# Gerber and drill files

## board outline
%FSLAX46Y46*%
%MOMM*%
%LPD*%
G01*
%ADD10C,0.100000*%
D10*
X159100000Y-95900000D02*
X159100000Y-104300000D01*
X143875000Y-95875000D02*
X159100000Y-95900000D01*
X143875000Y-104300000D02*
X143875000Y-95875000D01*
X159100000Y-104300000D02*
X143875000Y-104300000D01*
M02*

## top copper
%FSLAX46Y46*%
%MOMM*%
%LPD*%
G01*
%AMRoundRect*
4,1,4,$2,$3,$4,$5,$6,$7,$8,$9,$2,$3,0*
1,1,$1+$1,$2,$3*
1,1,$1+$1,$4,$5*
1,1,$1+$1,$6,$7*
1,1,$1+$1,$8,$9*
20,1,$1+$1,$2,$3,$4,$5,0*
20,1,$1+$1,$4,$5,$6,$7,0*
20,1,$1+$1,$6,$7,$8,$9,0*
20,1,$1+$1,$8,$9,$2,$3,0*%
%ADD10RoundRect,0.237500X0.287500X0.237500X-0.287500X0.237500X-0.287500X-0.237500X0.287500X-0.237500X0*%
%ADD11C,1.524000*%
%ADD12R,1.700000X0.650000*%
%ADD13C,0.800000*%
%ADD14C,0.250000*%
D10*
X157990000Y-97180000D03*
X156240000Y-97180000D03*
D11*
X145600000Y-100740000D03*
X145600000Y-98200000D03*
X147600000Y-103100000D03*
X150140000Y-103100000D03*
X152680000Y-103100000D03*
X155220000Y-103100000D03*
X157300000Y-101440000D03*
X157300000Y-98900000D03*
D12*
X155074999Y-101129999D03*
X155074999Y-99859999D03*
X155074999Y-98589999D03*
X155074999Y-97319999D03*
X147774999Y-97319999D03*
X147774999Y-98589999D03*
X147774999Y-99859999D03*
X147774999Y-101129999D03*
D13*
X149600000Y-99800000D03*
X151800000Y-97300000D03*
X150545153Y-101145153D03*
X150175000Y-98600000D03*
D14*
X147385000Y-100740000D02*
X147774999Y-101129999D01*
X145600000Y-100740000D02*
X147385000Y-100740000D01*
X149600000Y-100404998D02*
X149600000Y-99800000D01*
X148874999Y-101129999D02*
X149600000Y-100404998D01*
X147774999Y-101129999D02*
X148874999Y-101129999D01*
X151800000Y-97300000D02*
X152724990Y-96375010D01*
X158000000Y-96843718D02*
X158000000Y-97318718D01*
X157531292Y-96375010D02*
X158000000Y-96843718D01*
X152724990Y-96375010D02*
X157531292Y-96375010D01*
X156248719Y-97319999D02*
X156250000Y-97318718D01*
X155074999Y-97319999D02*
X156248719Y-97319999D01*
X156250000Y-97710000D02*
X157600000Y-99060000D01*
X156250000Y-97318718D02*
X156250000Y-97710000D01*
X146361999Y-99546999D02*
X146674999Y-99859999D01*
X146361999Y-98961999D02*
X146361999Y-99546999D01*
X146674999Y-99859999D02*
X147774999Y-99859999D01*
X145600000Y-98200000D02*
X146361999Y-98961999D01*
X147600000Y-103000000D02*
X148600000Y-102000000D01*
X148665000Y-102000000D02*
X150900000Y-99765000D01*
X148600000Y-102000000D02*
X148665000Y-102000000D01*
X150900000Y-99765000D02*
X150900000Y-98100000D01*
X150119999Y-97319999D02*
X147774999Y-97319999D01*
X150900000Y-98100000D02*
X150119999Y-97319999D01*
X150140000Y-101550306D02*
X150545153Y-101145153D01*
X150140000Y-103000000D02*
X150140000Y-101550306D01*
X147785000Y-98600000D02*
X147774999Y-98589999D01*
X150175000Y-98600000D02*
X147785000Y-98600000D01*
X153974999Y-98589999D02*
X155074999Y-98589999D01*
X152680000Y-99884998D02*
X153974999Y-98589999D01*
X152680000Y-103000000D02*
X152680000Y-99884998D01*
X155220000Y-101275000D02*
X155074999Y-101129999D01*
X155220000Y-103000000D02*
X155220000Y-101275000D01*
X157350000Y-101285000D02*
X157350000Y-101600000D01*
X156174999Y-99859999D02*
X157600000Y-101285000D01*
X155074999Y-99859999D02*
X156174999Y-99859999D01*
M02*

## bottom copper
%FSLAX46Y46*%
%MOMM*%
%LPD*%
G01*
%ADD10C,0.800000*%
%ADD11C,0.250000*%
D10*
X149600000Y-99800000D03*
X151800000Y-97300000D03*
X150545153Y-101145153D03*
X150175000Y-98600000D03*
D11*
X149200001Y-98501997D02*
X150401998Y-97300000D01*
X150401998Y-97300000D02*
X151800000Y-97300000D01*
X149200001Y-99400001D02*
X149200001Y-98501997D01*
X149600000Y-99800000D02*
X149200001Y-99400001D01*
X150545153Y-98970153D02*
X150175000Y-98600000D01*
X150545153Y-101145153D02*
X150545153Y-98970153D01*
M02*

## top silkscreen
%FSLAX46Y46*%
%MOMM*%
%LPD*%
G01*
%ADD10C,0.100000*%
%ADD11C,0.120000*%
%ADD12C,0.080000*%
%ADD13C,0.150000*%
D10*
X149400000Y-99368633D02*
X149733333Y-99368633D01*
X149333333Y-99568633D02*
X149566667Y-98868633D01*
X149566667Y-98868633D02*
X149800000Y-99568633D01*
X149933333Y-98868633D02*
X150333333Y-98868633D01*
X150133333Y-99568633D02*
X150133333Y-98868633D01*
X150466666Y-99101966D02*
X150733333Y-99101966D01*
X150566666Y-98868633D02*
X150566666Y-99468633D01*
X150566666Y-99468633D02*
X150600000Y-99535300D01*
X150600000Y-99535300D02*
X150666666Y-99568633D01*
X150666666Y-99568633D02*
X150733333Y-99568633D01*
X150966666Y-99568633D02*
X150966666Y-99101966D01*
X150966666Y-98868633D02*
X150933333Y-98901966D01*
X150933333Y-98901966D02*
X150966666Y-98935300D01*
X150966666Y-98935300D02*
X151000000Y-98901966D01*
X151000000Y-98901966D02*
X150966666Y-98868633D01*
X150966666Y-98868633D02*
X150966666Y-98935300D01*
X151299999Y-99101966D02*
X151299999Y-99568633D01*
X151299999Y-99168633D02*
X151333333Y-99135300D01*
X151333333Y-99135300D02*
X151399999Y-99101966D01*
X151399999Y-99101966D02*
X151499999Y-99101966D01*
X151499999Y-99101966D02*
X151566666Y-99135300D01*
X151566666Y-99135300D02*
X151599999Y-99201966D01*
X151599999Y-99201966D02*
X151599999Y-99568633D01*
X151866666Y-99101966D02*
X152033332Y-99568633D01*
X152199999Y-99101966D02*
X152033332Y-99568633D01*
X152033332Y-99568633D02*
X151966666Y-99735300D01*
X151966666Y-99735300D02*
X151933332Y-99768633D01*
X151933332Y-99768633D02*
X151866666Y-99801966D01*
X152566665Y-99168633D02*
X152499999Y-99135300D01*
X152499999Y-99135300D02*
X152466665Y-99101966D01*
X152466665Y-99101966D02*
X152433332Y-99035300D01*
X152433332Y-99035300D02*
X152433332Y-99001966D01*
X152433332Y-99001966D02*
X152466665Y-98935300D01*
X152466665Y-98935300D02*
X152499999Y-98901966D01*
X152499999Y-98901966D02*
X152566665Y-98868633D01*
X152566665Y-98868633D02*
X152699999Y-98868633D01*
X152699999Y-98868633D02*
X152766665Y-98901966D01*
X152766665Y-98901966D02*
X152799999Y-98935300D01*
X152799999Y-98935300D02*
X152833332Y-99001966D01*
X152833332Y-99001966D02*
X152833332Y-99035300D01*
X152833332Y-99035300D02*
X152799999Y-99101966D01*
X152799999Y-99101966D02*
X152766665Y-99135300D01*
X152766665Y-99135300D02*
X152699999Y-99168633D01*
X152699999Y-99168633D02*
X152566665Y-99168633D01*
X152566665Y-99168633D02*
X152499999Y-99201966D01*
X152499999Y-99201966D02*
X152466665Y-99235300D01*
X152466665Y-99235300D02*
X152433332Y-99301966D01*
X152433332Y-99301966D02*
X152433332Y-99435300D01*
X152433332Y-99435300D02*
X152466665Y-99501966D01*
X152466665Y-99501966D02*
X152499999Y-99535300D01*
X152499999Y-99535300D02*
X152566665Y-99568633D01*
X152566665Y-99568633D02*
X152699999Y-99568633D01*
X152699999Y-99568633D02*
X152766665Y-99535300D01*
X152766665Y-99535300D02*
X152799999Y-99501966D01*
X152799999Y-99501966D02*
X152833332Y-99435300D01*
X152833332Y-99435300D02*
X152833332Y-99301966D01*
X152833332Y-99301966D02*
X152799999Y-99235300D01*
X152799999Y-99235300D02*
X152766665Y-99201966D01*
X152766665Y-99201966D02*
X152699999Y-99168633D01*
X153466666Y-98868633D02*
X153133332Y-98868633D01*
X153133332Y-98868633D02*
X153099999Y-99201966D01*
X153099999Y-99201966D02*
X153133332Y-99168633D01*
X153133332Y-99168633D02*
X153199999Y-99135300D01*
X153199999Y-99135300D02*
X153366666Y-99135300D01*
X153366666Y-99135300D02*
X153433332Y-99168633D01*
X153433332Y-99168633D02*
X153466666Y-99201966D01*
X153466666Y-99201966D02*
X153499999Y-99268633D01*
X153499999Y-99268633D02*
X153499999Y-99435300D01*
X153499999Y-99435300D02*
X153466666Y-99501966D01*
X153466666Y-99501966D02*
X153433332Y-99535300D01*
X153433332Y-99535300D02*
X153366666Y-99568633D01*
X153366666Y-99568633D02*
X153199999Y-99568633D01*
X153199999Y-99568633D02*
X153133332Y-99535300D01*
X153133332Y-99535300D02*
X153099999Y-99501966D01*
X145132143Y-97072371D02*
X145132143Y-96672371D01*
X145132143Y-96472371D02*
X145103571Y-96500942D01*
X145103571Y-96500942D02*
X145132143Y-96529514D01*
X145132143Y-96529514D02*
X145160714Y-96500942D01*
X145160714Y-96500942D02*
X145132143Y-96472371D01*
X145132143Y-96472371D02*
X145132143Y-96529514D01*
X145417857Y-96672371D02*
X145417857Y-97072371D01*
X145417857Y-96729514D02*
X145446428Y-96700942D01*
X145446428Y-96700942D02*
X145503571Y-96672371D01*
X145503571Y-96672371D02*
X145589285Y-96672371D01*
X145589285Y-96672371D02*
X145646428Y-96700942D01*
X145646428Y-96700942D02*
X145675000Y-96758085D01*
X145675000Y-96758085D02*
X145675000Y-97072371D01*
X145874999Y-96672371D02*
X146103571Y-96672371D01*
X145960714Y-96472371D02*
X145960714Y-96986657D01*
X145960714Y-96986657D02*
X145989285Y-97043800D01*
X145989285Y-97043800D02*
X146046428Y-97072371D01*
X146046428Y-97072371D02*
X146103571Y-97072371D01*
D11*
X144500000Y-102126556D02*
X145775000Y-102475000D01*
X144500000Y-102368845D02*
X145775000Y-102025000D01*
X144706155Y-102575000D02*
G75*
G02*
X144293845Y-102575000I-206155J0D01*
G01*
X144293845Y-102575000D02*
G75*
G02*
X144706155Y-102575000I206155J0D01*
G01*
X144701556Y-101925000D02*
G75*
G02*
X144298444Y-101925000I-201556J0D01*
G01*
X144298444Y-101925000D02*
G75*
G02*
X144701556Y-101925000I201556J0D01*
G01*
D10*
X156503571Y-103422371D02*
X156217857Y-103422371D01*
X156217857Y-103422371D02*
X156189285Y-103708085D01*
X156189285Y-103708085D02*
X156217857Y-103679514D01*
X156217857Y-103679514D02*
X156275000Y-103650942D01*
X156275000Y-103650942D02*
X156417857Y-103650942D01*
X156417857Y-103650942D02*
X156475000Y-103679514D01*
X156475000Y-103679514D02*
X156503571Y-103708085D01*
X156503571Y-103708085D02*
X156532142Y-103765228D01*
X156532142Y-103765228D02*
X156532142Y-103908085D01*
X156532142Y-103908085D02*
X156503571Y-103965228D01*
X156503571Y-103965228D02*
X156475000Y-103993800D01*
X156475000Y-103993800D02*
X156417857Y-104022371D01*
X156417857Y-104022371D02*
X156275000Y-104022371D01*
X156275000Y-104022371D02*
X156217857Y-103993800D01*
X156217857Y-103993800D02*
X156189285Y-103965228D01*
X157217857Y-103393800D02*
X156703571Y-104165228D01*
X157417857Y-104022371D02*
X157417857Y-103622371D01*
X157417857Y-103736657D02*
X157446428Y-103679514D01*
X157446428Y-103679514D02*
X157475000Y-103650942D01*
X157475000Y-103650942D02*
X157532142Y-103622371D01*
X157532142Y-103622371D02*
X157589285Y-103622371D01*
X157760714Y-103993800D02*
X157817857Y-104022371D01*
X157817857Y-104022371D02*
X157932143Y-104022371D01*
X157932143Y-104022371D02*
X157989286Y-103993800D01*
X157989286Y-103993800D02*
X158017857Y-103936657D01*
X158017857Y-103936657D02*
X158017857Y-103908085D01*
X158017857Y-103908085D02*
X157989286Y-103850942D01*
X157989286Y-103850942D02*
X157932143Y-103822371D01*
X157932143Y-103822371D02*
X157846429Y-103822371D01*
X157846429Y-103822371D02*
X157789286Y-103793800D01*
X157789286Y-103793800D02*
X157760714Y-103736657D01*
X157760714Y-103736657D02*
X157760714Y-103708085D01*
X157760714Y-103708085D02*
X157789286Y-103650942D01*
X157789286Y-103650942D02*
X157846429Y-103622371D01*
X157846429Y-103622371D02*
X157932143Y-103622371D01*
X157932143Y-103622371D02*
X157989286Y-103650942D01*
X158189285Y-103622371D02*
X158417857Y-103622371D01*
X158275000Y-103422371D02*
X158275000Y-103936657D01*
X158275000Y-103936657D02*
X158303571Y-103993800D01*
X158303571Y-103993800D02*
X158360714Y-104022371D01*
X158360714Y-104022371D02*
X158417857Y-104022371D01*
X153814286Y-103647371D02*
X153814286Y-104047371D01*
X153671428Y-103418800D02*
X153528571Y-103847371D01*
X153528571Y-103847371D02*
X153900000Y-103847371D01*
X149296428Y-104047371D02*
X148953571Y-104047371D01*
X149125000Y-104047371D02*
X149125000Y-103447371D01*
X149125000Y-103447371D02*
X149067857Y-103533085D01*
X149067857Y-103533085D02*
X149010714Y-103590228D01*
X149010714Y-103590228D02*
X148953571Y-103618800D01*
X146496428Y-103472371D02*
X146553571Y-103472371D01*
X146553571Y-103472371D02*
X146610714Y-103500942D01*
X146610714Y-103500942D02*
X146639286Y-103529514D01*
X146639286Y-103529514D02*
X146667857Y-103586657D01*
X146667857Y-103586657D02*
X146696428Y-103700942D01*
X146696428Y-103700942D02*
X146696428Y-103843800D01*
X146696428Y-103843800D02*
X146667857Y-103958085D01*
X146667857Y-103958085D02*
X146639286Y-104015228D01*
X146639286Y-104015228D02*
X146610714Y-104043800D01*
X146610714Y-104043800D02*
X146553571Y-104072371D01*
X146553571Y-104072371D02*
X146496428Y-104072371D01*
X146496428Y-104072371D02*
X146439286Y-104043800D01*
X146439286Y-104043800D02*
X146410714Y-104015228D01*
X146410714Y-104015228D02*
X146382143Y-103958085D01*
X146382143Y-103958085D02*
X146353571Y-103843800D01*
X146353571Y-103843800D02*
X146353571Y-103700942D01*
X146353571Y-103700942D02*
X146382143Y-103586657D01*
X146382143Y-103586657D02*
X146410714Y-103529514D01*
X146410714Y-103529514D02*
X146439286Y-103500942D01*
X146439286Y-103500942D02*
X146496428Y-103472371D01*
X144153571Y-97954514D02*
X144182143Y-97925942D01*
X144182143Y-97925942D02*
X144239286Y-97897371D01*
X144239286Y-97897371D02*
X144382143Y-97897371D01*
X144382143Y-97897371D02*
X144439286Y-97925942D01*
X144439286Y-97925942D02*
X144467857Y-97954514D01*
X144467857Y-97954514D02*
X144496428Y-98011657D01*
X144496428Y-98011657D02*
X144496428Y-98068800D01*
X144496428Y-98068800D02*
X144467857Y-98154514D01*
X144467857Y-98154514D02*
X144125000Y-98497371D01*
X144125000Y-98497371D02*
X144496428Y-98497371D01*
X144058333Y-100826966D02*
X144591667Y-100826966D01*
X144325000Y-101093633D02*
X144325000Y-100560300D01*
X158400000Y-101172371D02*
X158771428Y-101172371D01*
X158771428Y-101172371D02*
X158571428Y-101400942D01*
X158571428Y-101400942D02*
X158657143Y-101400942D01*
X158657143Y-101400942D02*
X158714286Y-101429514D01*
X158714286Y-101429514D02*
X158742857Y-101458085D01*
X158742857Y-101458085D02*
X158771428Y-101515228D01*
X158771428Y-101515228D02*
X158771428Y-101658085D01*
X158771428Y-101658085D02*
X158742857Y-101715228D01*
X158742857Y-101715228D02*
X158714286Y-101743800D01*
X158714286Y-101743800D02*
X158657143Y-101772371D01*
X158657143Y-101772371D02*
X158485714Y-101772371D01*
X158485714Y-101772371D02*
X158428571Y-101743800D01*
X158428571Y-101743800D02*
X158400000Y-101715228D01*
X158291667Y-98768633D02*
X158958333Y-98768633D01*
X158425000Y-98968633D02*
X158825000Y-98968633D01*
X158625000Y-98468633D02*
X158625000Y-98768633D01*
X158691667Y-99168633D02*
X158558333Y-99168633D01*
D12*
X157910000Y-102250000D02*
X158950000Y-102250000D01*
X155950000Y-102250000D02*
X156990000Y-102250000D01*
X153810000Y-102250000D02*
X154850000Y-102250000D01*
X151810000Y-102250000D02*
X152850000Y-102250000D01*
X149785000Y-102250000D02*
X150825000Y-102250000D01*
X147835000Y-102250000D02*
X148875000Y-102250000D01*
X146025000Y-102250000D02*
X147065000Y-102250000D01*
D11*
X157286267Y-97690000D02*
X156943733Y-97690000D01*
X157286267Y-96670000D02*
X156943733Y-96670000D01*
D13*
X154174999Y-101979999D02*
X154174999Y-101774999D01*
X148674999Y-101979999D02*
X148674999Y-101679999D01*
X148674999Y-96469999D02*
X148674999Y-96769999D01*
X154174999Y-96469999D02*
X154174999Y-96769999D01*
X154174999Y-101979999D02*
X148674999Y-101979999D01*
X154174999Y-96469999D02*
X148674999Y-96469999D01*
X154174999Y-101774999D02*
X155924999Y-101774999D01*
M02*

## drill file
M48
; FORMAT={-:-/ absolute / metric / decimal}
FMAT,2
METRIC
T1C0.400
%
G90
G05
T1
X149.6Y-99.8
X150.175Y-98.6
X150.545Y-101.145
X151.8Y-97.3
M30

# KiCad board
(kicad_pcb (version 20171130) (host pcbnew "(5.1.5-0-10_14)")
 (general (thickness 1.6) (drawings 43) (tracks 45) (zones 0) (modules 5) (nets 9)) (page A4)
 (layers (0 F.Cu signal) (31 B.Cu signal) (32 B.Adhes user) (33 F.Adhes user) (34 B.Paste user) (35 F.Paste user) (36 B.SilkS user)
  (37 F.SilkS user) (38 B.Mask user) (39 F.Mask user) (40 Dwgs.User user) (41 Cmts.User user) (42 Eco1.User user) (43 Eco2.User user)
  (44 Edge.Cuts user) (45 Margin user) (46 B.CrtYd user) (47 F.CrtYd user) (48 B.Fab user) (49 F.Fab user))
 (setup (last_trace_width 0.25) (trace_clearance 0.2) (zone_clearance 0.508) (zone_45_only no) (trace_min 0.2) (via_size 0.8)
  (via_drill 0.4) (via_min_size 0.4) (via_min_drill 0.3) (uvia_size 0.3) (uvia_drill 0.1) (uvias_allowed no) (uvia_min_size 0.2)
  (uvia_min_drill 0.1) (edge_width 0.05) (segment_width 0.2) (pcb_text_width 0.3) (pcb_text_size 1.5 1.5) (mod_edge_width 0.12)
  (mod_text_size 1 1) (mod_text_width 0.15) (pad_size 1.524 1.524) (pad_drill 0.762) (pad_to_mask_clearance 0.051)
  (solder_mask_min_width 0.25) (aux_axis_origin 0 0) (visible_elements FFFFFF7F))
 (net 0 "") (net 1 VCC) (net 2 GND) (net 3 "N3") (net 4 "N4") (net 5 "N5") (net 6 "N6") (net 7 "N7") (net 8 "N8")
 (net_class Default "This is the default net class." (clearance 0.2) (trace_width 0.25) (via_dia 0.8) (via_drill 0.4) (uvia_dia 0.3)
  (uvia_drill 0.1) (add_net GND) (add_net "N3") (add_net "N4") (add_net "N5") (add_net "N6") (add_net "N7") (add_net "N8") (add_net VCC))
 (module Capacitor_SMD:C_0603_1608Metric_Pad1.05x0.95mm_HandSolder (layer F.Cu) (at 157.115 97.18 180)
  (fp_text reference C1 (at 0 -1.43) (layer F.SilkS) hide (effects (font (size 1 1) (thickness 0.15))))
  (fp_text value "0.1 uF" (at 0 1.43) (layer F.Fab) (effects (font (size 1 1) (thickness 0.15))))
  (fp_line (start -0.171267 -0.51) (end 0.171267 -0.51) (layer F.SilkS) (width 0.12))
  (fp_line (start -0.171267 0.51) (end 0.171267 0.51) (layer F.SilkS) (width 0.12))
  (pad 1 smd roundrect (at -0.875 0 180) (size 1.05 0.95) (layers F.Cu F.Paste F.Mask) (roundrect_rratio 0.25) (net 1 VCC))
  (pad 2 smd roundrect (at 0.875 0 180) (size 1.05 0.95) (layers F.Cu F.Paste F.Mask) (roundrect_rratio 0.25) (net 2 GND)))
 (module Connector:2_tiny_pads (layer F.Cu) (at 143.06 99.47 90)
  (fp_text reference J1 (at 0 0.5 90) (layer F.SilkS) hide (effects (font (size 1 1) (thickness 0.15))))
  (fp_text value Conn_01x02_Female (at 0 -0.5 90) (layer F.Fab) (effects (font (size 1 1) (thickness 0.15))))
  (pad 1 smd circle (at -1.27 2.54 90) (size 1.524 1.524) (layers F.Cu F.Paste F.Mask) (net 1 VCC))
  (pad 2 smd circle (at 1.27 2.54 90) (size 1.524 1.524) (layers F.Cu F.Paste F.Mask) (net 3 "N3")))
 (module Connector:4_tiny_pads (layer F.Cu) (at 151.41 100.56)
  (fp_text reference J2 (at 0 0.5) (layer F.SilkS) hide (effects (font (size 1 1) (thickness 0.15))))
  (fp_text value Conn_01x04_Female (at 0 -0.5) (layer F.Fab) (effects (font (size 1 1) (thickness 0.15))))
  (pad 1 smd circle (at -3.81 2.54) (size 1.524 1.524) (layers F.Cu F.Paste F.Mask) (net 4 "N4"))
  (pad 2 smd circle (at -1.27 2.54) (size 1.524 1.524) (layers F.Cu F.Paste F.Mask) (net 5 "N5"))
  (pad 3 smd circle (at 1.27 2.54) (size 1.524 1.524) (layers F.Cu F.Paste F.Mask) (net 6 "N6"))
  (pad 4 smd circle (at 3.81 2.54) (size 1.524 1.524) (layers F.Cu F.Paste F.Mask) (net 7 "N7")))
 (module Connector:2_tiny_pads (layer F.Cu) (at 159.84 100.17 270)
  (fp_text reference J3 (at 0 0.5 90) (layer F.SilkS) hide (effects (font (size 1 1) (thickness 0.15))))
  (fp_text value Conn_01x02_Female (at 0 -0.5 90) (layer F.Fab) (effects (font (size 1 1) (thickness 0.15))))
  (pad 2 smd circle (at 1.27 2.54 270) (size 1.524 1.524) (layers F.Cu F.Paste F.Mask) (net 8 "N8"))
  (pad 1 smd circle (at -1.27 2.54 270) (size 1.524 1.524) (layers F.Cu F.Paste F.Mask) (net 2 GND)))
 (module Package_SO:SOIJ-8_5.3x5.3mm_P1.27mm (layer F.Cu) (at 151.424999 99.224999 180)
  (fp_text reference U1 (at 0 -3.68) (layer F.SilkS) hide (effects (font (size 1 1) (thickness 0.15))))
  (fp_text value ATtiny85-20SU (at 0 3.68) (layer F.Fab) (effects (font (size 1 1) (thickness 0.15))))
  (fp_line (start -2.75 -2.755) (end -2.75 -2.55) (layer F.SilkS) (width 0.15))
  (fp_line (start 2.75 -2.755) (end 2.75 -2.455) (layer F.SilkS) (width 0.15))
  (fp_line (start 2.75 2.755) (end 2.75 2.455) (layer F.SilkS) (width 0.15))
  (fp_line (start -2.75 2.755) (end -2.75 2.455) (layer F.SilkS) (width 0.15))
  (fp_line (start -2.75 -2.755) (end 2.75 -2.755) (layer F.SilkS) (width 0.15))
  (fp_line (start -2.75 2.755) (end 2.75 2.755) (layer F.SilkS) (width 0.15))
  (fp_line (start -2.75 -2.55) (end -4.5 -2.55) (layer F.SilkS) (width 0.15))
  (pad 1 smd rect (at -3.65 -1.905 180) (size 1.7 0.65) (layers F.Cu F.Paste F.Mask) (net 7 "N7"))
  (pad 2 smd rect (at -3.65 -0.635 180) (size 1.7 0.65) (layers F.Cu F.Paste F.Mask) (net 8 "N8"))
  (pad 3 smd rect (at -3.65 0.635 180) (size 1.7 0.65) (layers F.Cu F.Paste F.Mask) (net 6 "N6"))
  (pad 4 smd rect (at -3.65 1.905 180) (size 1.7 0.65) (layers F.Cu F.Paste F.Mask) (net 2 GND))
  (pad 5 smd rect (at 3.65 1.905 180) (size 1.7 0.65) (layers F.Cu F.Paste F.Mask) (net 4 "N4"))
  (pad 6 smd rect (at 3.65 0.635 180) (size 1.7 0.65) (layers F.Cu F.Paste F.Mask) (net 5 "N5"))
  (pad 7 smd rect (at 3.65 -0.635 180) (size 1.7 0.65) (layers F.Cu F.Paste F.Mask) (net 3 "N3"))
  (pad 8 smd rect (at 3.65 -1.905 180) (size 1.7 0.65) (layers F.Cu F.Paste F.Mask) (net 1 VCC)))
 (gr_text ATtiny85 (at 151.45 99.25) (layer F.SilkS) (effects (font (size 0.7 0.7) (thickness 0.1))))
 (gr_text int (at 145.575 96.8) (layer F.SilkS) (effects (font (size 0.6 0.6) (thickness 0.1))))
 (gr_line (start 144.5 102.126556) (end 145.775 102.475) (layer F.SilkS) (width 0.12))
 (gr_line (start 144.5 102.368845) (end 145.775 102.025) (layer F.SilkS) (width 0.12))
 (gr_circle (center 144.5 102.575) (end 144.55 102.375) (layer F.SilkS) (width 0.12))
 (gr_circle (center 144.5 101.925) (end 144.6 102.1) (layer F.SilkS) (width 0.12))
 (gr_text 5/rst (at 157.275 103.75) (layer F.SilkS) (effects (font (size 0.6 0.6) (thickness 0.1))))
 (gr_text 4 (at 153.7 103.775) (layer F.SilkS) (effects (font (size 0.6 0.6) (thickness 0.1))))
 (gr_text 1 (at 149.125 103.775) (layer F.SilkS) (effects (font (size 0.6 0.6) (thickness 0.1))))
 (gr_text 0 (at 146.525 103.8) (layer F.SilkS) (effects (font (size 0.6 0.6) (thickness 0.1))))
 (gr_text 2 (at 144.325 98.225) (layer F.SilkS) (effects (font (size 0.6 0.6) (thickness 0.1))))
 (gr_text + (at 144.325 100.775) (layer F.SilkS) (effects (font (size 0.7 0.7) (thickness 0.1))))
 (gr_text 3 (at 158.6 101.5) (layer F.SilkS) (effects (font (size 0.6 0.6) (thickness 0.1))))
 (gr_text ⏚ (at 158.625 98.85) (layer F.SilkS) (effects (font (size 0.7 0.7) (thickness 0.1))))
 (gr_line (start 157.91 102.25) (end 158.95 102.25) (layer F.SilkS) (width 0.08))
 (gr_line (start 155.95 102.25) (end 156.99 102.25) (layer F.SilkS) (width 0.08))
 (gr_line (start 153.81 102.25) (end 154.85 102.25) (layer F.SilkS) (width 0.08))
 (gr_line (start 151.81 102.25) (end 152.85 102.25) (layer F.SilkS) (width 0.08))
 (gr_line (start 149.785 102.25) (end 150.825 102.25) (layer F.SilkS) (width 0.08))
 (gr_line (start 147.835 102.25) (end 148.875 102.25) (layer F.SilkS) (width 0.08))
 (gr_line (start 146.025 102.25) (end 147.065 102.25) (layer F.SilkS) (width 0.08))
 (gr_line (start 159.1 95.9) (end 159.1 104.3) (layer Edge.Cuts) (width 0.1))
 (gr_line (start 143.875 95.875) (end 159.1 95.9) (layer Edge.Cuts) (width 0.1))
 (gr_line (start 143.875 104.3) (end 143.875 95.875) (layer Edge.Cuts) (width 0.1))
 (gr_line (start 159.1 104.3) (end 143.875 104.3) (layer Edge.Cuts) (width 0.1))
 (segment (start 147.385 100.74) (end 147.774999 101.129999) (width 0.25) (layer F.Cu) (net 1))
 (segment (start 145.6 100.74) (end 147.385 100.74) (width 0.25) (layer F.Cu) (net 1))
 (via (at 149.6 99.8) (size 0.8) (drill 0.4) (layers F.Cu B.Cu) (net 1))
 (segment (start 149.6 100.404998) (end 149.6 99.8) (width 0.25) (layer F.Cu) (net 1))
 (segment (start 148.874999 101.129999) (end 149.6 100.404998) (width 0.25) (layer F.Cu) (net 1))
 (segment (start 147.774999 101.129999) (end 148.874999 101.129999) (width 0.25) (layer F.Cu) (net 1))
 (via (at 151.8 97.3) (size 0.8) (drill 0.4) (layers F.Cu B.Cu) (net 1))
 (segment (start 149.200001 98.501997) (end 150.401998 97.3) (width 0.25) (layer B.Cu) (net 1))
 (segment (start 150.401998 97.3) (end 151.8 97.3) (width 0.25) (layer B.Cu) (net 1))
 (segment (start 149.200001 99.400001) (end 149.200001 98.501997) (width 0.25) (layer B.Cu) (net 1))
 (segment (start 149.6 99.8) (end 149.200001 99.400001) (width 0.25) (layer B.Cu) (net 1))
 (segment (start 151.8 97.3) (end 152.72499 96.37501) (width 0.25) (layer F.Cu) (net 1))
 (segment (start 158 96.843718) (end 158 97.318718) (width 0.25) (layer F.Cu) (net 1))
 (segment (start 157.531292 96.37501) (end 158 96.843718) (width 0.25) (layer F.Cu) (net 1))
 (segment (start 152.72499 96.37501) (end 157.531292 96.37501) (width 0.25) (layer F.Cu) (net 1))
 (segment (start 156.248719 97.319999) (end 156.25 97.318718) (width 0.25) (layer F.Cu) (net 2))
 (segment (start 155.074999 97.319999) (end 156.248719 97.319999) (width 0.25) (layer F.Cu) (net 2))
 (segment (start 156.25 97.71) (end 157.6 99.06) (width 0.25) (layer F.Cu) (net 2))
 (segment (start 156.25 97.318718) (end 156.25 97.71) (width 0.25) (layer F.Cu) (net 2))
 (segment (start 146.361999 99.546999) (end 146.674999 99.859999) (width 0.25) (layer F.Cu) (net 3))
 (segment (start 146.361999 98.961999) (end 146.361999 99.546999) (width 0.25) (layer F.Cu) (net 3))
 (segment (start 146.674999 99.859999) (end 147.774999 99.859999) (width 0.25) (layer F.Cu) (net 3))
 (segment (start 145.6 98.2) (end 146.361999 98.961999) (width 0.25) (layer F.Cu) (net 3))
 (segment (start 147.6 103) (end 148.6 102) (width 0.25) (layer F.Cu) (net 4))
 (segment (start 148.665 102) (end 150.9 99.765) (width 0.25) (layer F.Cu) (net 4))
 (segment (start 148.6 102) (end 148.665 102) (width 0.25) (layer F.Cu) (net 4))
 (segment (start 150.9 99.765) (end 150.9 98.1) (width 0.25) (layer F.Cu) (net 4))
 (segment (start 150.119999 97.319999) (end 147.774999 97.319999) (width 0.25) (layer F.Cu) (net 4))
 (segment (start 150.9 98.1) (end 150.119999 97.319999) (width 0.25) (layer F.Cu) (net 4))
 (via (at 150.545153 101.145153) (size 0.8) (drill 0.4) (layers F.Cu B.Cu) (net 5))
 (segment (start 150.14 101.550306) (end 150.545153 101.145153) (width 0.25) (layer F.Cu) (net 5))
 (segment (start 150.14 103) (end 150.14 101.550306) (width 0.25) (layer F.Cu) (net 5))
 (via (at 150.175 98.6) (size 0.8) (drill 0.4) (layers F.Cu B.Cu) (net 5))
 (segment (start 150.545153 98.970153) (end 150.175 98.6) (width 0.25) (layer B.Cu) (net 5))
 (segment (start 150.545153 101.145153) (end 150.545153 98.970153) (width 0.25) (layer B.Cu) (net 5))
 (segment (start 147.785 98.6) (end 147.774999 98.589999) (width 0.25) (layer F.Cu) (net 5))
 (segment (start 150.175 98.6) (end 147.785 98.6) (width 0.25) (layer F.Cu) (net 5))
 (segment (start 153.974999 98.589999) (end 155.074999 98.589999) (width 0.25) (layer F.Cu) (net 6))
 (segment (start 152.68 99.884998) (end 153.974999 98.589999) (width 0.25) (layer F.Cu) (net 6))
 (segment (start 152.68 103) (end 152.68 99.884998) (width 0.25) (layer F.Cu) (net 6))
 (segment (start 155.22 101.275) (end 155.074999 101.129999) (width 0.25) (layer F.Cu) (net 7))
 (segment (start 155.22 103) (end 155.22 101.275) (width 0.25) (layer F.Cu) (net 7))
 (segment (start 157.35 101.285) (end 157.35 101.6) (width 0.25) (layer F.Cu) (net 8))
 (segment (start 156.174999 99.859999) (end 157.6 101.285) (width 0.25) (layer F.Cu) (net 8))
 (segment (start 155.074999 99.859999) (end 156.174999 99.859999) (width 0.25) (layer F.Cu) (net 8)))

